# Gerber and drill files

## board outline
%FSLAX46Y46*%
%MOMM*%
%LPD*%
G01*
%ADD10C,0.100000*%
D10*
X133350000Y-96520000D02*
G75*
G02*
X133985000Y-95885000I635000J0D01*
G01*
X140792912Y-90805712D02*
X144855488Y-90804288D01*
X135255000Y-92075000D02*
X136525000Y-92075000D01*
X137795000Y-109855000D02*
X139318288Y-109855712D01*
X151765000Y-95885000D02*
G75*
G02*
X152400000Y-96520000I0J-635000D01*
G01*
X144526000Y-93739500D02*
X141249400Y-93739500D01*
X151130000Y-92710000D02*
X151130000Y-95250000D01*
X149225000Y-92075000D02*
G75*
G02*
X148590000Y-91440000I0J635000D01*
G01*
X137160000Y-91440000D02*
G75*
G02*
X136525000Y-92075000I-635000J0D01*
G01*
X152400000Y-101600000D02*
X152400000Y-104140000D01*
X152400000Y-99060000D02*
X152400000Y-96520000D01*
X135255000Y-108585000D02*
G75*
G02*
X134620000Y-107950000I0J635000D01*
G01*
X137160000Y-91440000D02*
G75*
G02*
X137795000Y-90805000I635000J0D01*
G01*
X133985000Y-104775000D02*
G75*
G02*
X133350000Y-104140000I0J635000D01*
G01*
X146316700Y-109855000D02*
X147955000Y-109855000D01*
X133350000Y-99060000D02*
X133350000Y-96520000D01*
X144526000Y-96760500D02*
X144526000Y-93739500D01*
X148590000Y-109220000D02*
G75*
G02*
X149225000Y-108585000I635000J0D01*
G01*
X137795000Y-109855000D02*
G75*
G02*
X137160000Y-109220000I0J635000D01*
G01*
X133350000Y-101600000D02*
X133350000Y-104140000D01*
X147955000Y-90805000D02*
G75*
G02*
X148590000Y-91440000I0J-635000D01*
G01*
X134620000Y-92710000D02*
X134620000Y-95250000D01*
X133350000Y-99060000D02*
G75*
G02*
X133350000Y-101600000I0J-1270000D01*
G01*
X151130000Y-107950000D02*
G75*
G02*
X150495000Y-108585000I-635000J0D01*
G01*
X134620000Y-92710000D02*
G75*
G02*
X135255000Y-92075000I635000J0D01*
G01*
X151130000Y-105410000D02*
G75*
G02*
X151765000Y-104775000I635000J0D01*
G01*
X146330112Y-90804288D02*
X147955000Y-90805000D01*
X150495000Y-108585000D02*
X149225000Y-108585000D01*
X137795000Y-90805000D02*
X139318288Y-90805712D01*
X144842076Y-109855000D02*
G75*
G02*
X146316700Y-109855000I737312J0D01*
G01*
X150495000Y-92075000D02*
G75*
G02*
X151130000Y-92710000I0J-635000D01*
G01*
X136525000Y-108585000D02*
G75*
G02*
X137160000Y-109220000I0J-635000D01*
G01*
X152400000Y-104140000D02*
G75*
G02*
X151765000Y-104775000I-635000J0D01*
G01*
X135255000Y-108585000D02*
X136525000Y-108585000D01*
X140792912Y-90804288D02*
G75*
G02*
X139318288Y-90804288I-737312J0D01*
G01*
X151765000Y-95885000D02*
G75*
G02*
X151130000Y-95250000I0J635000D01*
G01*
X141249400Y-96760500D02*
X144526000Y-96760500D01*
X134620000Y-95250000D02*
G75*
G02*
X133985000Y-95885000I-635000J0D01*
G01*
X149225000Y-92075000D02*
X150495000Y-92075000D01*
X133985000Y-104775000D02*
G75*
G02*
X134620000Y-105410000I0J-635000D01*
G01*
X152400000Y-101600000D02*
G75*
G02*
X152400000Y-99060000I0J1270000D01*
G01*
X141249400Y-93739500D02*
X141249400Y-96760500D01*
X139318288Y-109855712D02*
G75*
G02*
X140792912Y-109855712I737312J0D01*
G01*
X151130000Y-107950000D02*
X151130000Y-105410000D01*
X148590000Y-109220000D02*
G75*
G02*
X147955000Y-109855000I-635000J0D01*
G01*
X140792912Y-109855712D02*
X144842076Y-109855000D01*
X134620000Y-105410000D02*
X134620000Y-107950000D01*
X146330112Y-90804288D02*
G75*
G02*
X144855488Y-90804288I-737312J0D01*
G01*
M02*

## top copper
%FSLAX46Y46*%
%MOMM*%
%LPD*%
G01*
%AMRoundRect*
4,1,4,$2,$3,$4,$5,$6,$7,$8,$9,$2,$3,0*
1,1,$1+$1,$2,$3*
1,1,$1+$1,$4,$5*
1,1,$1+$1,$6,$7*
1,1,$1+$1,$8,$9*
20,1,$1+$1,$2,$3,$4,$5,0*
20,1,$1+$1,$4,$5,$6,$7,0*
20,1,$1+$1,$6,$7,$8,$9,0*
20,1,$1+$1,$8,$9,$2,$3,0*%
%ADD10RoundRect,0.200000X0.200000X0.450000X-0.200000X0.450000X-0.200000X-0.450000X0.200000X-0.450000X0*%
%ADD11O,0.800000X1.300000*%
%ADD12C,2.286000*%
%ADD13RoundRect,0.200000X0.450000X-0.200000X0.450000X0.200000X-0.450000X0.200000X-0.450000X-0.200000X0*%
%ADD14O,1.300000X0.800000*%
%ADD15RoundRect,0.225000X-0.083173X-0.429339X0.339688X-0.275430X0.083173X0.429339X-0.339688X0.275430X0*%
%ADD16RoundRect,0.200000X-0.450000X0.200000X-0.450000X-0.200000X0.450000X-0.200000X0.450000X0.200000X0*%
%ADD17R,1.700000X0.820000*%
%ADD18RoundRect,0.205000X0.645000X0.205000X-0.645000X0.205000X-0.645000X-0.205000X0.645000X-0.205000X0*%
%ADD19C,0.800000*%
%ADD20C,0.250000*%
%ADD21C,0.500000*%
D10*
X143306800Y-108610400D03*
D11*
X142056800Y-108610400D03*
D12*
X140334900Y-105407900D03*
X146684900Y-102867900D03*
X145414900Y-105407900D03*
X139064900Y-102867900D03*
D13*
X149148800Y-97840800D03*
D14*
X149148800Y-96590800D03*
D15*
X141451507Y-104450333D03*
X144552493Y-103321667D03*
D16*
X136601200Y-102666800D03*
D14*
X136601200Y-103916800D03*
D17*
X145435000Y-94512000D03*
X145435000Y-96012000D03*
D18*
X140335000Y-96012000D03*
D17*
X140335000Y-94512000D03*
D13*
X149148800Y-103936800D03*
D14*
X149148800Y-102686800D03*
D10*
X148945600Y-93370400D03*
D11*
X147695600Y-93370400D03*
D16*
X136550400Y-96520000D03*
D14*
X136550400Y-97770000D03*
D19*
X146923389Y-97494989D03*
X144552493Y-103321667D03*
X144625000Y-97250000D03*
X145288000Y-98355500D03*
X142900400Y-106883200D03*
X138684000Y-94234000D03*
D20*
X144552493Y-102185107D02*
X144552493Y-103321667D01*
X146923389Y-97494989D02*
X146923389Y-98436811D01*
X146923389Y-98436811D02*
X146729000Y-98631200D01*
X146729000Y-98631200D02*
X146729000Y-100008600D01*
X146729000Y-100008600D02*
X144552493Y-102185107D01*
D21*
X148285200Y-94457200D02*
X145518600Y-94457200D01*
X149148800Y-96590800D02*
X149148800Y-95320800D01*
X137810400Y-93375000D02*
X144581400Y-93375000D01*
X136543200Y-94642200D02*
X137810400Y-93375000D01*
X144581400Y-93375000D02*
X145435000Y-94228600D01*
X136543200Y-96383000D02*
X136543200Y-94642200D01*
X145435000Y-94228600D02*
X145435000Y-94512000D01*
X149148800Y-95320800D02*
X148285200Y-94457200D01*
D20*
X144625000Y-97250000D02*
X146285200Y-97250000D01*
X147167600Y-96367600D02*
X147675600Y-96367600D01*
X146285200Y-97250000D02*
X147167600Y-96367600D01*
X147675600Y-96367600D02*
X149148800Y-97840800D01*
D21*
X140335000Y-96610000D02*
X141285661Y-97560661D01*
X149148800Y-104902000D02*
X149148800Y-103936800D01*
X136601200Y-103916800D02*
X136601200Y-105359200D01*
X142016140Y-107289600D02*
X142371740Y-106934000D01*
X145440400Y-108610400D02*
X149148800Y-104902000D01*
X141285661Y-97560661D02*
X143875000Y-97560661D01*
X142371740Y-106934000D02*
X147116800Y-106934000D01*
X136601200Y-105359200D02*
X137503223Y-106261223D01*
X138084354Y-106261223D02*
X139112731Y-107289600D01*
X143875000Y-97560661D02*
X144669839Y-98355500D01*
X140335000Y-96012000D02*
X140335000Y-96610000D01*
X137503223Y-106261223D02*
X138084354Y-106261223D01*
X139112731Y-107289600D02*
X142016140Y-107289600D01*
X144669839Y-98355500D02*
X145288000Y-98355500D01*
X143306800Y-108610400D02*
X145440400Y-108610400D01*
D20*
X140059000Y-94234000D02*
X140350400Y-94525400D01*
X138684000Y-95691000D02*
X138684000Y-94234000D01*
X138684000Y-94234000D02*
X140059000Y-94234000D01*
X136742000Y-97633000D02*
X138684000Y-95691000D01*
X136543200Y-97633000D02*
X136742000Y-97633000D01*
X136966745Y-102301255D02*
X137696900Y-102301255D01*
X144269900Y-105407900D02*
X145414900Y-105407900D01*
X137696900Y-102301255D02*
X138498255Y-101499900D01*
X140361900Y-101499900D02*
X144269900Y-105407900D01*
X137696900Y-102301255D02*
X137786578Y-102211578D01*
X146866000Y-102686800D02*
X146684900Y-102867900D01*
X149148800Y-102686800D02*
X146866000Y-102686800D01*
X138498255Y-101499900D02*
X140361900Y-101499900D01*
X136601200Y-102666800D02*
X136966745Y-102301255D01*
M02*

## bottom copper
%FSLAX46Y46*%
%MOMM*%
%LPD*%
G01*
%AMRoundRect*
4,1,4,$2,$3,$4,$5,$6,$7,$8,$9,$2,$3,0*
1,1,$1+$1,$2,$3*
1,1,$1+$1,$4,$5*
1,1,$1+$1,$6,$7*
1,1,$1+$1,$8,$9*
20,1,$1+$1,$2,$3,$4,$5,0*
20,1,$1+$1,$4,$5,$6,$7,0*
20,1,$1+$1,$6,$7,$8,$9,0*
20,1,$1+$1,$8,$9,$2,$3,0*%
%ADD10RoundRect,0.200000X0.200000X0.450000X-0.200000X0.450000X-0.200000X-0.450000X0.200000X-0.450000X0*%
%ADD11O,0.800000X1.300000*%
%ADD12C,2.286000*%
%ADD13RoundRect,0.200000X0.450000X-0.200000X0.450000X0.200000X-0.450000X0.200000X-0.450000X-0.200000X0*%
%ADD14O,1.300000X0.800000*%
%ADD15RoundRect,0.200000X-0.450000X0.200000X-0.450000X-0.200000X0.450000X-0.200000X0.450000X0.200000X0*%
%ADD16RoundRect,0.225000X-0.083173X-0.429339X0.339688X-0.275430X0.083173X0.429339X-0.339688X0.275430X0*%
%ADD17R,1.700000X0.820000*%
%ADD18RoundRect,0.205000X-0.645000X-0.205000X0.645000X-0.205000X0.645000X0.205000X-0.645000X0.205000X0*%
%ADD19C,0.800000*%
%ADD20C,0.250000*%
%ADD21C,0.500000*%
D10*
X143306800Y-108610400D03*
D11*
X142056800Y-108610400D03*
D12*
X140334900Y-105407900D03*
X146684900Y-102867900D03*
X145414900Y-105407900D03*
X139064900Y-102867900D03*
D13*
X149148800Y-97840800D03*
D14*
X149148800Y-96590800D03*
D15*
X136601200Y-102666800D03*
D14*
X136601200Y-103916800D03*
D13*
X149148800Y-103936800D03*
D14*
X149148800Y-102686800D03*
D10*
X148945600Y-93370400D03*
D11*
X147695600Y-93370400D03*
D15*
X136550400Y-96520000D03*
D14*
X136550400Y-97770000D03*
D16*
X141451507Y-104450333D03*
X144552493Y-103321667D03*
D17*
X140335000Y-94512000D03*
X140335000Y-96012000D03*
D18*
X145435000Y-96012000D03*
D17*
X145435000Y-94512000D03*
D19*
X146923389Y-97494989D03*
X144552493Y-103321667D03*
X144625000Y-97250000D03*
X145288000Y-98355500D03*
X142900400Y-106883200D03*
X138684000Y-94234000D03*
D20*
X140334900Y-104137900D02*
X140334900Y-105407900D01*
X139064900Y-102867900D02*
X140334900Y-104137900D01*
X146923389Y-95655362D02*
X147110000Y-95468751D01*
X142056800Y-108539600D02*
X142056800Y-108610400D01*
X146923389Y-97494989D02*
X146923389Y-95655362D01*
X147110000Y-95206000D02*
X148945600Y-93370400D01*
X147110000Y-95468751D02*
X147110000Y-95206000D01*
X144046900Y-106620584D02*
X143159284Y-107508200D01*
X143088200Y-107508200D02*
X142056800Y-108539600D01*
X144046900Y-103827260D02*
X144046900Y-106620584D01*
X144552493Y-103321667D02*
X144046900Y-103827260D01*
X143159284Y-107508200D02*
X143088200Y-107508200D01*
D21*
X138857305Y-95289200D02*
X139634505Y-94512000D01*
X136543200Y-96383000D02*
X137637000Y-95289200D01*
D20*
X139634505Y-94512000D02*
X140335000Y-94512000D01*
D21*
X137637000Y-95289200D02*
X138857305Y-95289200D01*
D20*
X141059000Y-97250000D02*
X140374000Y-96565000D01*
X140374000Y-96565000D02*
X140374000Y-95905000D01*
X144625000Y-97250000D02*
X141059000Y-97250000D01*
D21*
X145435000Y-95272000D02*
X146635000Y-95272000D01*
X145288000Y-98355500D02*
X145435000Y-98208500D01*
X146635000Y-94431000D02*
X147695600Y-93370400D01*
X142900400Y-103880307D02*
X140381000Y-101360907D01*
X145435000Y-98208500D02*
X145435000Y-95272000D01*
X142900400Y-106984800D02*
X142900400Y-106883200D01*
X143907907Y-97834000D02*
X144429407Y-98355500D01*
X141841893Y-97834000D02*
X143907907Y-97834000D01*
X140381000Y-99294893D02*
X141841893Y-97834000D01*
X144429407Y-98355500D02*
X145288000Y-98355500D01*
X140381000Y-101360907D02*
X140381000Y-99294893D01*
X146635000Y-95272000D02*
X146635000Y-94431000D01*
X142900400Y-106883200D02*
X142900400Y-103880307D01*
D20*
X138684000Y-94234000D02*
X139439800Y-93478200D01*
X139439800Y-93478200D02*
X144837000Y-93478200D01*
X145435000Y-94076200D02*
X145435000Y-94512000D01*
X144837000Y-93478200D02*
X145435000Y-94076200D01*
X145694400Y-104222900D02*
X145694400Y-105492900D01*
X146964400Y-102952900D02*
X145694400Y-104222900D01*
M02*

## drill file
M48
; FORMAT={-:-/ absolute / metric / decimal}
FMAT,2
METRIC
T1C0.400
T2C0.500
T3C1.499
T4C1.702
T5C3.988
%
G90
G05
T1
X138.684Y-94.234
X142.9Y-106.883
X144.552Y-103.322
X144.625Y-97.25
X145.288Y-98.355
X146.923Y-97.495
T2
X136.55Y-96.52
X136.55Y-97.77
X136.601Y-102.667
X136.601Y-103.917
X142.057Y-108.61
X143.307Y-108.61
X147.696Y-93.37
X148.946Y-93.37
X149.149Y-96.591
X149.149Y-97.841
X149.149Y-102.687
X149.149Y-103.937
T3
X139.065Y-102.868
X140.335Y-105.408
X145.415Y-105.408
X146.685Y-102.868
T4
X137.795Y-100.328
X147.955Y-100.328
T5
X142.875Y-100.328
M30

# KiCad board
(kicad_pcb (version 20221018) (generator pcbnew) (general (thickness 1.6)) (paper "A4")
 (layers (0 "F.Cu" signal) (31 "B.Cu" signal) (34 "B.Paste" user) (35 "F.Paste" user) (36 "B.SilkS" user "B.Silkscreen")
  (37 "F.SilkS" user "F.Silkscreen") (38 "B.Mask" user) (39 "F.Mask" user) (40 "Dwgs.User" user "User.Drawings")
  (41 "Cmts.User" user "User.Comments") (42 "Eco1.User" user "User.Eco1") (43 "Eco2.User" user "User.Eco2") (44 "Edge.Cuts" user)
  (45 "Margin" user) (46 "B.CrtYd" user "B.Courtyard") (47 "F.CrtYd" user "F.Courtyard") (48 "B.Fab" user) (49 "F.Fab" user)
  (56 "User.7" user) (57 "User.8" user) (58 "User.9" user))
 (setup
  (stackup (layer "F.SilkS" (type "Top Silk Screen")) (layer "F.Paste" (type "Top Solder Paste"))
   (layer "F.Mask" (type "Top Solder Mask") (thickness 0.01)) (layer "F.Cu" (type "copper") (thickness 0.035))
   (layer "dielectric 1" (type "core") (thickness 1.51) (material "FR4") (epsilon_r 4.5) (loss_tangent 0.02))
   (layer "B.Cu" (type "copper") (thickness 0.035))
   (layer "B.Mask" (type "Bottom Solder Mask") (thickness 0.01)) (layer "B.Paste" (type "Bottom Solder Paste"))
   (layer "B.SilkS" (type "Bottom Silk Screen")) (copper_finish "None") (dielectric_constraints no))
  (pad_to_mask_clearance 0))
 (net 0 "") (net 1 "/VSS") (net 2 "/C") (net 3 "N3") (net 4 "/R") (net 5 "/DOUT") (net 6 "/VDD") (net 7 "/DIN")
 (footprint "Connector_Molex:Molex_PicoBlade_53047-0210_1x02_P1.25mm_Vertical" (layer "F.Cu") (at 143.3068 108.6104 180)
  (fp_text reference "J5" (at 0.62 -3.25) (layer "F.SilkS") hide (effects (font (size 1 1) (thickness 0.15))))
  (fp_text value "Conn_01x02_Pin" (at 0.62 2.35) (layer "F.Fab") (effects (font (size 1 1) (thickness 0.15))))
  (pad "1" thru_hole roundrect (at 0 0 180) (size 0.8 1.3) (drill 0.5) (layers "*.Cu" "*.Mask") (roundrect_rratio 0.25) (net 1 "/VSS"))
  (pad "2" thru_hole oval (at 1.25 0 180) (size 0.8 1.3) (drill 0.5) (layers "*.Cu" "*.Mask") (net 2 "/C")))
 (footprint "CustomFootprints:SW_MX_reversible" (layer "F.Cu") (at 142.8749 100.3279 180)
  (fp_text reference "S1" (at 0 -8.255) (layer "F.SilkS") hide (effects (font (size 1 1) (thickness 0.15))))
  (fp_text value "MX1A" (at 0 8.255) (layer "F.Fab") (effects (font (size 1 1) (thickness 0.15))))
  (pad "" np_thru_hole circle (at -5.08 0 180) (size 1.7018 1.7018) (drill 1.7018) (layers "*.Cu" "*.Mask"))
  (pad "" np_thru_hole circle (at 0 0 180) (size 3.9878 3.9878) (drill 3.9878) (layers "*.Cu" "*.Mask"))
  (pad "" thru_hole circle (at 2.54 -5.08 180) (size 2.286 2.286) (drill 1.4986) (layers "*.Cu" "*.Mask") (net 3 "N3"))
  (pad "" np_thru_hole circle (at 5.08 0 180) (size 1.7018 1.7018) (drill 1.7018) (layers "*.Cu" "*.Mask"))
  (pad "1" thru_hole circle (at -3.81 -2.54 180) (size 2.286 2.286) (drill 1.4986) (layers "*.Cu" "*.Mask") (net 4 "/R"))
  (pad "1" thru_hole circle (at -2.54 -5.08 180) (size 2.286 2.286) (drill 1.4986) (layers "*.Cu" "*.Mask") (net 4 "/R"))
  (pad "2" thru_hole circle (at 3.81 -2.54 180) (size 2.286 2.286) (drill 1.4986) (layers "*.Cu" "*.Mask") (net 3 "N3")))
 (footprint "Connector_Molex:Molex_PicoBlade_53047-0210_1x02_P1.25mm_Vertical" (layer "F.Cu") (at 149.1488 97.8408 90)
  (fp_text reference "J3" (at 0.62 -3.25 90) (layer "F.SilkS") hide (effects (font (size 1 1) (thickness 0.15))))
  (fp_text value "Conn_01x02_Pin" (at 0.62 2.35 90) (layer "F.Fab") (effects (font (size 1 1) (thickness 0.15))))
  (pad "1" thru_hole roundrect (at 0 0 90) (size 0.8 1.3) (drill 0.5) (layers "*.Cu" "*.Mask") (roundrect_rratio 0.25) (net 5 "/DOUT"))
  (pad "2" thru_hole oval (at 1.25 0 90) (size 0.8 1.3) (drill 0.5) (layers "*.Cu" "*.Mask") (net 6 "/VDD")))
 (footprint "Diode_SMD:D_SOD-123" (layer "F.Cu") (at 143.002 103.886 20)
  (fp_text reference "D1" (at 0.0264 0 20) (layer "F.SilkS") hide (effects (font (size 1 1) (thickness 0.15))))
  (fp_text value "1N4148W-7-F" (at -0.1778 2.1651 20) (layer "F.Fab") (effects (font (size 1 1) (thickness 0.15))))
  (pad "1" smd roundrect (at -1.65 0 20) (size 0.9 1.2) (layers "F.Cu" "F.Paste" "F.Mask") (roundrect_rratio 0.25) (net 3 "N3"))
  (pad "2" smd roundrect (at 1.65 0 20) (size 0.9 1.2) (layers "F.Cu" "F.Paste" "F.Mask") (roundrect_rratio 0.25) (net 2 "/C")))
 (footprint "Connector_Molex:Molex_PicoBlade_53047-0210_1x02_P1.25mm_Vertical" (layer "F.Cu") (at 136.6012 102.6668 -90)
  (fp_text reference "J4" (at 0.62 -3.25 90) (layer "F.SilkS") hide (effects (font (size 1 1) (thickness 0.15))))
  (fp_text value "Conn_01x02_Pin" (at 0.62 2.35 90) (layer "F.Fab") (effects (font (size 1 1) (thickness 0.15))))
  (pad "1" thru_hole roundrect (at 0 0 270) (size 0.8 1.3) (drill 0.5) (layers "*.Cu" "*.Mask") (roundrect_rratio 0.25) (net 4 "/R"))
  (pad "2" thru_hole oval (at 1.25 0 270) (size 0.8 1.3) (drill 0.5) (layers "*.Cu" "*.Mask") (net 1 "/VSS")))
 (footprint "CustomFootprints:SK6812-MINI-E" (layer "F.Cu") (at 142.885 95.262 180)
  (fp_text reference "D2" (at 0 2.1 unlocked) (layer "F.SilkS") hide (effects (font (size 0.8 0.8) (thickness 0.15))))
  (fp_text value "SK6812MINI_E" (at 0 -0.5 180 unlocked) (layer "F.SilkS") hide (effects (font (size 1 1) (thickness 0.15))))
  (pad "1" smd rect (at -2.55 0.75 180) (size 1.7 0.82) (layers "F.Cu" "F.Paste" "F.Mask") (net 6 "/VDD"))
  (pad "2" smd rect (at -2.55 -0.75 180) (size 1.7 0.82) (layers "F.Cu" "F.Paste" "F.Mask") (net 5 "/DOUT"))
  (pad "3" smd roundrect (at 2.55 -0.75 180) (size 1.7 0.82) (layers "F.Cu" "F.Paste" "F.Mask") (roundrect_rratio 0.25) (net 1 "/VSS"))
  (pad "4" smd rect (at 2.55 0.75 180) (size 1.7 0.82) (layers "F.Cu" "F.Paste" "F.Mask") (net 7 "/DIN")))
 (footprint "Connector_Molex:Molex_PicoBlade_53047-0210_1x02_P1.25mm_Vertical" (layer "F.Cu") (at 149.1488 103.9368 90)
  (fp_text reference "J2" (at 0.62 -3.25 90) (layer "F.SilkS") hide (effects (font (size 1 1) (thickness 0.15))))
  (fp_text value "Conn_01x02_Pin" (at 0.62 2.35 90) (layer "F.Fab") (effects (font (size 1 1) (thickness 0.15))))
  (pad "1" thru_hole roundrect (at 0 0 90) (size 0.8 1.3) (drill 0.5) (layers "*.Cu" "*.Mask") (roundrect_rratio 0.25) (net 1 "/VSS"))
  (pad "2" thru_hole oval (at 1.25 0 90) (size 0.8 1.3) (drill 0.5) (layers "*.Cu" "*.Mask") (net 4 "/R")))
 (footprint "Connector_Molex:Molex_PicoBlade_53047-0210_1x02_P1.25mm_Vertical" (layer "F.Cu") (at 148.9456 93.3704 180)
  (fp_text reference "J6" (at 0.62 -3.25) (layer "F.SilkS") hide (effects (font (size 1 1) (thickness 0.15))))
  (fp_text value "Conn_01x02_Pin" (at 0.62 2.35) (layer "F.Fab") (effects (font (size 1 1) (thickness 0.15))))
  (pad "1" thru_hole roundrect (at 0 0 180) (size 0.8 1.3) (drill 0.5) (layers "*.Cu" "*.Mask") (roundrect_rratio 0.25) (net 2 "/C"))
  (pad "2" thru_hole oval (at 1.25 0 180) (size 0.8 1.3) (drill 0.5) (layers "*.Cu" "*.Mask") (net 1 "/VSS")))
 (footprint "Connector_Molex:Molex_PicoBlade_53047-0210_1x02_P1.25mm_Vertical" (layer "F.Cu") (at 136.5504 96.52 -90)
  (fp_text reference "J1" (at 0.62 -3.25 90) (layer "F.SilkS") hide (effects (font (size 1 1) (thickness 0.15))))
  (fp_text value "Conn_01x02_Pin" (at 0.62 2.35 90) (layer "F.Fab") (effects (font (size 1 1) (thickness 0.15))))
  (pad "1" thru_hole roundrect (at 0 0 270) (size 0.8 1.3) (drill 0.5) (layers "*.Cu" "*.Mask") (roundrect_rratio 0.25) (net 6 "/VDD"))
  (pad "2" thru_hole oval (at 1.25 0 270) (size 0.8 1.3) (drill 0.5) (layers "*.Cu" "*.Mask") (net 7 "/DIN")))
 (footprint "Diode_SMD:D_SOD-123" (layer "B.Cu") (at 143.002 103.886 20)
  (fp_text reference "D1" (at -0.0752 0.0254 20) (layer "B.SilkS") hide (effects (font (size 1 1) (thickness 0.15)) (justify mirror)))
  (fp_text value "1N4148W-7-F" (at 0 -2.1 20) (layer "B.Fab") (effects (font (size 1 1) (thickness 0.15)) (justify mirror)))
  (pad "1" smd roundrect (at -1.65 0 20) (size 0.9 1.2) (layers "B.Cu" "B.Paste" "B.Mask") (roundrect_rratio 0.25) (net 3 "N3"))
  (pad "2" smd roundrect (at 1.65 0 20) (size 0.9 1.2) (layers "B.Cu" "B.Paste" "B.Mask") (roundrect_rratio 0.25) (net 2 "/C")))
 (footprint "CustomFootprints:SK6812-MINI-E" (layer "B.Cu") (at 142.885 95.262)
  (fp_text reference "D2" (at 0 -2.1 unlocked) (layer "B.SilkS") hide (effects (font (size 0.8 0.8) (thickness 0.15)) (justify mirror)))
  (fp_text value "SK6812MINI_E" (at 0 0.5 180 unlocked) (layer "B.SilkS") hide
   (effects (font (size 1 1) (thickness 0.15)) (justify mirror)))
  (pad "1" smd rect (at -2.55 -0.75) (size 1.7 0.82) (layers "B.Cu" "B.Paste" "B.Mask") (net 6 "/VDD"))
  (pad "2" smd rect (at -2.55 0.75) (size 1.7 0.82) (layers "B.Cu" "B.Paste" "B.Mask") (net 5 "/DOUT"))
  (pad "3" smd roundrect (at 2.55 0.75) (size 1.7 0.82) (layers "B.Cu" "B.Paste" "B.Mask") (roundrect_rratio 0.25) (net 1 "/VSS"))
  (pad "4" smd rect (at 2.55 -0.75) (size 1.7 0.82) (layers "B.Cu" "B.Paste" "B.Mask") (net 7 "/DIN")))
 (gr_arc (start 133.35 96.52) (mid 133.535987 96.070987) (end 133.985 95.885) (stroke (width 0.1) (type solid)) (layer "Edge.Cuts"))
 (gr_line (start 140.792912 90.805712) (end 144.855488 90.804288) (stroke (width 0.1) (type solid)) (layer "Edge.Cuts"))
 (gr_line (start 135.255 92.075) (end 136.525 92.075) (stroke (width 0.1) (type solid)) (layer "Edge.Cuts"))
 (gr_line (start 137.795 109.855) (end 139.318288 109.855712) (stroke (width 0.1) (type solid)) (layer "Edge.Cuts"))
 (gr_arc (start 151.765 95.885) (mid 152.214013 96.070987) (end 152.4 96.52) (stroke (width 0.1) (type solid)) (layer "Edge.Cuts"))
 (gr_line (start 144.526 93.7395) (end 141.2494 93.7395) (stroke (width 0.1) (type solid)) (layer "Edge.Cuts"))
 (gr_line (start 151.13 92.71) (end 151.13 95.25) (stroke (width 0.1) (type solid)) (layer "Edge.Cuts"))
 (gr_arc (start 149.225 92.075) (mid 148.775987 91.889013) (end 148.59 91.44) (stroke (width 0.1) (type solid)) (layer "Edge.Cuts"))
 (gr_arc (start 137.16 91.44) (mid 136.974013 91.889013) (end 136.525 92.075) (stroke (width 0.1) (type solid)) (layer "Edge.Cuts"))
 (gr_line (start 152.4 101.6) (end 152.4 104.14) (stroke (width 0.1) (type solid)) (layer "Edge.Cuts"))
 (gr_line (start 152.4 99.06) (end 152.4 96.52) (stroke (width 0.1) (type solid)) (layer "Edge.Cuts"))
 (gr_arc (start 135.255 108.585) (mid 134.805987 108.399013) (end 134.62 107.95) (stroke (width 0.1) (type solid)) (layer "Edge.Cuts"))
 (gr_arc (start 137.16 91.44) (mid 137.345987 90.990987) (end 137.795 90.805) (stroke (width 0.1) (type solid)) (layer "Edge.Cuts"))
 (gr_arc (start 133.985 104.775) (mid 133.535987 104.589013) (end 133.35 104.14) (stroke (width 0.1) (type solid)) (layer "Edge.Cuts"))
 (gr_line (start 146.3167 109.855) (end 147.955 109.855) (stroke (width 0.1) (type solid)) (layer "Edge.Cuts"))
 (gr_line (start 133.35 99.06) (end 133.35 96.52) (stroke (width 0.1) (type solid)) (layer "Edge.Cuts"))
 (gr_line (start 144.526 96.7605) (end 144.526 93.7395) (stroke (width 0.1) (type solid)) (layer "Edge.Cuts"))
 (gr_arc (start 148.59 109.22) (mid 148.775987 108.770987) (end 149.225 108.585) (stroke (width 0.1) (type solid)) (layer "Edge.Cuts"))
 (gr_arc (start 137.795 109.855) (mid 137.345987 109.669013) (end 137.16 109.22) (stroke (width 0.1) (type solid)) (layer "Edge.Cuts"))
 (gr_line (start 133.35 101.6) (end 133.35 104.14) (stroke (width 0.1) (type solid)) (layer "Edge.Cuts"))
 (gr_arc (start 147.955 90.805) (mid 148.404013 90.990987) (end 148.59 91.44) (stroke (width 0.1) (type solid)) (layer "Edge.Cuts"))
 (gr_line (start 134.62 92.71) (end 134.62 95.25) (stroke (width 0.1) (type solid)) (layer "Edge.Cuts"))
 (gr_arc (start 133.35 99.06) (mid 134.62 100.33) (end 133.35 101.6) (stroke (width 0.1) (type solid)) (layer "Edge.Cuts"))
 (gr_arc (start 151.13 107.95) (mid 150.944013 108.399013) (end 150.495 108.585) (stroke (width 0.1) (type solid)) (layer "Edge.Cuts"))
 (gr_arc (start 134.62 92.71) (mid 134.805987 92.260987) (end 135.255 92.075) (stroke (width 0.1) (type solid)) (layer "Edge.Cuts"))
 (gr_arc (start 151.13 105.41) (mid 151.315987 104.960987) (end 151.765 104.775) (stroke (width 0.1) (type solid)) (layer "Edge.Cuts"))
 (gr_line (start 146.330112 90.804288) (end 147.955 90.805) (stroke (width 0.1) (type solid)) (layer "Edge.Cuts"))
 (gr_line (start 150.495 108.585) (end 149.225 108.585) (stroke (width 0.1) (type solid)) (layer "Edge.Cuts"))
 (gr_line (start 137.795 90.805) (end 139.318288 90.805712) (stroke (width 0.1) (type solid)) (layer "Edge.Cuts"))
 (gr_arc (start 144.842076 109.855) (mid 145.579388 109.117688) (end 146.3167 109.855) (stroke (width 0.1) (type solid)) (layer "Edge.Cuts"))
 (gr_arc (start 150.495 92.075) (mid 150.944013 92.260987) (end 151.13 92.71) (stroke (width 0.1) (type solid)) (layer "Edge.Cuts"))
 (gr_arc (start 136.525 108.585) (mid 136.974013 108.770987) (end 137.16 109.22) (stroke (width 0.1) (type solid)) (layer "Edge.Cuts"))
 (gr_arc (start 152.4 104.14) (mid 152.214013 104.589013) (end 151.765 104.775) (stroke (width 0.1) (type solid)) (layer "Edge.Cuts"))
 (gr_line (start 135.255 108.585) (end 136.525 108.585) (stroke (width 0.1) (type solid)) (layer "Edge.Cuts"))
 (gr_arc (start 140.792912 90.804288) (mid 140.0556 91.5416) (end 139.318288 90.804288) (stroke (width 0.1) (type solid))
  (layer "Edge.Cuts"))
 (gr_arc (start 151.765 95.885) (mid 151.315987 95.699013) (end 151.13 95.25) (stroke (width 0.1) (type solid)) (layer "Edge.Cuts"))
 (gr_line (start 141.2494 96.7605) (end 144.526 96.7605) (stroke (width 0.1) (type solid)) (layer "Edge.Cuts"))
 (gr_arc (start 134.62 95.25) (mid 134.434013 95.699013) (end 133.985 95.885) (stroke (width 0.1) (type solid)) (layer "Edge.Cuts"))
 (gr_line (start 149.225 92.075) (end 150.495 92.075) (stroke (width 0.1) (type solid)) (layer "Edge.Cuts"))
 (gr_arc (start 133.985 104.775) (mid 134.434013 104.960987) (end 134.62 105.41) (stroke (width 0.1) (type solid)) (layer "Edge.Cuts"))
 (gr_arc (start 152.4 101.6) (mid 151.13 100.33) (end 152.4 99.06) (stroke (width 0.1) (type solid)) (layer "Edge.Cuts"))
 (gr_line (start 141.2494 93.7395) (end 141.2494 96.7605) (stroke (width 0.1) (type solid)) (layer "Edge.Cuts"))
 (gr_arc (start 139.318288 109.855712) (mid 140.0556 109.1184) (end 140.792912 109.855712) (stroke (width 0.1) (type solid))
  (layer "Edge.Cuts"))
 (gr_line (start 151.13 107.95) (end 151.13 105.41) (stroke (width 0.1) (type solid)) (layer "Edge.Cuts"))
 (gr_arc (start 148.59 109.22) (mid 148.404013 109.669013) (end 147.955 109.855) (stroke (width 0.1) (type solid)) (layer "Edge.Cuts"))
 (gr_line (start 140.792912 109.855712) (end 144.842076 109.855) (stroke (width 0.1) (type solid)) (layer "Edge.Cuts"))
 (gr_line (start 134.62 105.41) (end 134.62 107.95) (stroke (width 0.1) (type solid)) (layer "Edge.Cuts"))
 (gr_arc (start 146.330112 90.804288) (mid 145.5928 91.5416) (end 144.855488 90.804288) (stroke (width 0.1) (type solid))
  (layer "Edge.Cuts"))
 (segment (start 140.3349 104.1379) (end 140.3349 105.4079) (width 0.25) (layer "B.Cu") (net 3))
 (segment (start 139.0649 102.8679) (end 140.3349 104.1379) (width 0.25) (layer "B.Cu") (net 3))
 (segment (start 144.552493 102.185107) (end 144.552493 103.321667) (width 0.25) (layer "F.Cu") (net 2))
 (segment (start 146.923389 97.494989) (end 146.923389 98.436811) (width 0.25) (layer "F.Cu") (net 2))
 (segment (start 146.923389 98.436811) (end 146.729 98.6312) (width 0.25) (layer "F.Cu") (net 2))
 (segment (start 146.729 98.6312) (end 146.729 100.0086) (width 0.25) (layer "F.Cu") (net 2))
 (segment (start 146.729 100.0086) (end 144.552493 102.185107) (width 0.25) (layer "F.Cu") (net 2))
 (via (at 146.923389 97.494989) (size 0.8) (drill 0.4) (layers "F.Cu" "B.Cu") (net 2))
 (via (at 144.552493 103.321667) (size 0.8) (drill 0.4) (layers "F.Cu" "B.Cu") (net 2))
 (segment (start 146.923389 95.655362) (end 147.11 95.468751) (width 0.25) (layer "B.Cu") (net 2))
 (segment (start 142.0568 108.5396) (end 142.0568 108.6104) (width 0.25) (layer "B.Cu") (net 2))
 (segment (start 146.923389 97.494989) (end 146.923389 95.655362) (width 0.25) (layer "B.Cu") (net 2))
 (segment (start 147.11 95.206) (end 148.9456 93.3704) (width 0.25) (layer "B.Cu") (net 2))
 (segment (start 147.11 95.468751) (end 147.11 95.206) (width 0.25) (layer "B.Cu") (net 2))
 (segment (start 144.0469 106.620584) (end 143.159284 107.5082) (width 0.25) (layer "B.Cu") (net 2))
 (segment (start 143.0882 107.5082) (end 142.0568 108.5396) (width 0.25) (layer "B.Cu") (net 2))
 (segment (start 144.0469 103.82726) (end 144.0469 106.620584) (width 0.25) (layer "B.Cu") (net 2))
 (segment (start 144.552493 103.321667) (end 144.0469 103.82726) (width 0.25) (layer "B.Cu") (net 2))
 (segment (start 143.159284 107.5082) (end 143.0882 107.5082) (width 0.25) (layer "B.Cu") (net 2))
 (segment (start 148.2852 94.4572) (end 145.5186 94.4572) (width 0.5) (layer "F.Cu") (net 6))
 (segment (start 149.1488 96.5908) (end 149.1488 95.3208) (width 0.5) (layer "F.Cu") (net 6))
 (segment (start 137.8104 93.375) (end 144.5814 93.375) (width 0.5) (layer "F.Cu") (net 6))
 (segment (start 136.5432 94.6422) (end 137.8104 93.375) (width 0.5) (layer "F.Cu") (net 6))
 (segment (start 144.5814 93.375) (end 145.435 94.2286) (width 0.5) (layer "F.Cu") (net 6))
 (segment (start 136.5432 96.383) (end 136.5432 94.6422) (width 0.5) (layer "F.Cu") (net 6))
 (segment (start 145.435 94.2286) (end 145.435 94.512) (width 0.5) (layer "F.Cu") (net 6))
 (segment (start 149.1488 95.3208) (end 148.2852 94.4572) (width 0.5) (layer "F.Cu") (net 6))
 (segment (start 138.857305 95.2892) (end 139.634505 94.512) (width 0.5) (layer "B.Cu") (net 6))
 (segment (start 136.5432 96.383) (end 137.637 95.2892) (width 0.5) (layer "B.Cu") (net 6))
 (segment (start 139.634505 94.512) (end 140.335 94.512) (width 0.25) (layer "B.Cu") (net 6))
 (segment (start 137.637 95.2892) (end 138.857305 95.2892) (width 0.5) (layer "B.Cu") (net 6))
 (segment (start 144.625 97.25) (end 146.2852 97.25) (width 0.25) (layer "F.Cu") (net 5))
 (segment (start 147.1676 96.3676) (end 147.6756 96.3676) (width 0.25) (layer "F.Cu") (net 5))
 (segment (start 146.2852 97.25) (end 147.1676 96.3676) (width 0.25) (layer "F.Cu") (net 5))
 (segment (start 147.6756 96.3676) (end 149.1488 97.8408) (width 0.25) (layer "F.Cu") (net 5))
 (via (at 144.625 97.25) (size 0.8) (drill 0.4) (layers "F.Cu" "B.Cu") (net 5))
 (segment (start 141.059 97.25) (end 140.374 96.565) (width 0.25) (layer "B.Cu") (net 5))
 (segment (start 140.374 96.565) (end 140.374 95.905) (width 0.25) (layer "B.Cu") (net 5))
 (segment (start 144.625 97.25) (end 141.059 97.25) (width 0.25) (layer "B.Cu") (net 5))
 (segment (start 140.335 96.61) (end 141.285661 97.560661) (width 0.5) (layer "F.Cu") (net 1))
 (segment (start 149.1488 104.902) (end 149.1488 103.9368) (width 0.5) (layer "F.Cu") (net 1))
 (segment (start 136.6012 103.9168) (end 136.6012 105.3592) (width 0.5) (layer "F.Cu") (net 1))
 (segment (start 142.01614 107.2896) (end 142.37174 106.934) (width 0.5) (layer "F.Cu") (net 1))
 (segment (start 145.4404 108.6104) (end 149.1488 104.902) (width 0.5) (layer "F.Cu") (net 1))
 (segment (start 141.285661 97.560661) (end 143.875 97.560661) (width 0.5) (layer "F.Cu") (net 1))
 (segment (start 142.37174 106.934) (end 147.1168 106.934) (width 0.5) (layer "F.Cu") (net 1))
 (segment (start 136.6012 105.3592) (end 137.503223 106.261223) (width 0.5) (layer "F.Cu") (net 1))
 (segment (start 138.084354 106.261223) (end 139.112731 107.2896) (width 0.5) (layer "F.Cu") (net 1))
 (segment (start 143.875 97.560661) (end 144.669839 98.3555) (width 0.5) (layer "F.Cu") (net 1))
 (segment (start 140.335 96.012) (end 140.335 96.61) (width 0.5) (layer "F.Cu") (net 1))
 (segment (start 137.503223 106.261223) (end 138.084354 106.261223) (width 0.5) (layer "F.Cu") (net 1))
 (segment (start 139.112731 107.2896) (end 142.01614 107.2896) (width 0.5) (layer "F.Cu") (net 1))
 (segment (start 144.669839 98.3555) (end 145.288 98.3555) (width 0.5) (layer "F.Cu") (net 1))
 (segment (start 143.3068 108.6104) (end 145.4404 108.6104) (width 0.5) (layer "F.Cu") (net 1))
 (via (at 145.288 98.3555) (size 0.8) (drill 0.4) (layers "F.Cu" "B.Cu") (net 1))
 (via (at 142.9004 106.8832) (size 0.8) (drill 0.4) (layers "F.Cu" "B.Cu") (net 1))
 (segment (start 145.435 95.272) (end 146.635 95.272) (width 0.5) (layer "B.Cu") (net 1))
 (segment (start 145.288 98.3555) (end 145.435 98.2085) (width 0.5) (layer "B.Cu") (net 1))
 (segment (start 146.635 94.431) (end 147.6956 93.3704) (width 0.5) (layer "B.Cu") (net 1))
 (segment (start 142.9004 103.880307) (end 140.381 101.360907) (width 0.5) (layer "B.Cu") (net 1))
 (segment (start 145.435 98.2085) (end 145.435 95.272) (width 0.5) (layer "B.Cu") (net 1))
 (segment (start 142.9004 106.9848) (end 142.9004 106.8832) (width 0.5) (layer "B.Cu") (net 1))
 (segment (start 143.907907 97.834) (end 144.429407 98.3555) (width 0.5) (layer "B.Cu") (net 1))
 (segment (start 141.841893 97.834) (end 143.907907 97.834) (width 0.5) (layer "B.Cu") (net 1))
 (segment (start 140.381 99.294893) (end 141.841893 97.834) (width 0.5) (layer "B.Cu") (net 1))
 (segment (start 144.429407 98.3555) (end 145.288 98.3555) (width 0.5) (layer "B.Cu") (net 1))
 (segment (start 140.381 101.360907) (end 140.381 99.294893) (width 0.5) (layer "B.Cu") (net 1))
 (segment (start 146.635 95.272) (end 146.635 94.431) (width 0.5) (layer "B.Cu") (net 1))
 (segment (start 142.9004 106.8832) (end 142.9004 103.880307) (width 0.5) (layer "B.Cu") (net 1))
 (segment (start 140.059 94.234) (end 140.3504 94.5254) (width 0.25) (layer "F.Cu") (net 7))
 (segment (start 138.684 95.691) (end 138.684 94.234) (width 0.25) (layer "F.Cu") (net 7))
 (segment (start 138.684 94.234) (end 140.059 94.234) (width 0.25) (layer "F.Cu") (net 7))
 (segment (start 136.742 97.633) (end 138.684 95.691) (width 0.25) (layer "F.Cu") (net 7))
 (segment (start 136.5432 97.633) (end 136.742 97.633) (width 0.25) (layer "F.Cu") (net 7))
 (via (at 138.684 94.234) (size 0.8) (drill 0.4) (layers "F.Cu" "B.Cu") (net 7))
 (segment (start 138.684 94.234) (end 139.4398 93.4782) (width 0.25) (layer "B.Cu") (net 7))
 (segment (start 139.4398 93.4782) (end 144.837 93.4782) (width 0.25) (layer "B.Cu") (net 7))
 (segment (start 145.435 94.0762) (end 145.435 94.512) (width 0.25) (layer "B.Cu") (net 7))
 (segment (start 144.837 93.4782) (end 145.435 94.0762) (width 0.25) (layer "B.Cu") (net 7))
 (segment (start 136.966745 102.301255) (end 137.6969 102.301255) (width 0.25) (layer "F.Cu") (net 4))
 (segment (start 144.2699 105.4079) (end 145.4149 105.4079) (width 0.25) (layer "F.Cu") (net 4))
 (segment (start 137.6969 102.301255) (end 138.498255 101.4999) (width 0.25) (layer "F.Cu") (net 4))
 (segment (start 140.3619 101.4999) (end 144.2699 105.4079) (width 0.25) (layer "F.Cu") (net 4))
 (segment (start 137.6969 102.301255) (end 137.786578 102.211578) (width 0.25) (layer "F.Cu") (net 4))
 (segment (start 146.866 102.6868) (end 146.6849 102.8679) (width 0.25) (layer "F.Cu") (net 4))
 (segment (start 149.1488 102.6868) (end 146.866 102.6868) (width 0.25) (layer "F.Cu") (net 4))
 (segment (start 138.498255 101.4999) (end 140.3619 101.4999) (width 0.25) (layer "F.Cu") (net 4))
 (segment (start 136.6012 102.6668) (end 136.966745 102.301255) (width 0.25) (layer "F.Cu") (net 4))
 (segment (start 145.6944 104.2229) (end 145.6944 105.4929) (width 0.25) (layer "B.Cu") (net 4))
 (segment (start 146.9644 102.9529) (end 145.6944 104.2229) (width 0.25) (layer "B.Cu") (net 4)))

